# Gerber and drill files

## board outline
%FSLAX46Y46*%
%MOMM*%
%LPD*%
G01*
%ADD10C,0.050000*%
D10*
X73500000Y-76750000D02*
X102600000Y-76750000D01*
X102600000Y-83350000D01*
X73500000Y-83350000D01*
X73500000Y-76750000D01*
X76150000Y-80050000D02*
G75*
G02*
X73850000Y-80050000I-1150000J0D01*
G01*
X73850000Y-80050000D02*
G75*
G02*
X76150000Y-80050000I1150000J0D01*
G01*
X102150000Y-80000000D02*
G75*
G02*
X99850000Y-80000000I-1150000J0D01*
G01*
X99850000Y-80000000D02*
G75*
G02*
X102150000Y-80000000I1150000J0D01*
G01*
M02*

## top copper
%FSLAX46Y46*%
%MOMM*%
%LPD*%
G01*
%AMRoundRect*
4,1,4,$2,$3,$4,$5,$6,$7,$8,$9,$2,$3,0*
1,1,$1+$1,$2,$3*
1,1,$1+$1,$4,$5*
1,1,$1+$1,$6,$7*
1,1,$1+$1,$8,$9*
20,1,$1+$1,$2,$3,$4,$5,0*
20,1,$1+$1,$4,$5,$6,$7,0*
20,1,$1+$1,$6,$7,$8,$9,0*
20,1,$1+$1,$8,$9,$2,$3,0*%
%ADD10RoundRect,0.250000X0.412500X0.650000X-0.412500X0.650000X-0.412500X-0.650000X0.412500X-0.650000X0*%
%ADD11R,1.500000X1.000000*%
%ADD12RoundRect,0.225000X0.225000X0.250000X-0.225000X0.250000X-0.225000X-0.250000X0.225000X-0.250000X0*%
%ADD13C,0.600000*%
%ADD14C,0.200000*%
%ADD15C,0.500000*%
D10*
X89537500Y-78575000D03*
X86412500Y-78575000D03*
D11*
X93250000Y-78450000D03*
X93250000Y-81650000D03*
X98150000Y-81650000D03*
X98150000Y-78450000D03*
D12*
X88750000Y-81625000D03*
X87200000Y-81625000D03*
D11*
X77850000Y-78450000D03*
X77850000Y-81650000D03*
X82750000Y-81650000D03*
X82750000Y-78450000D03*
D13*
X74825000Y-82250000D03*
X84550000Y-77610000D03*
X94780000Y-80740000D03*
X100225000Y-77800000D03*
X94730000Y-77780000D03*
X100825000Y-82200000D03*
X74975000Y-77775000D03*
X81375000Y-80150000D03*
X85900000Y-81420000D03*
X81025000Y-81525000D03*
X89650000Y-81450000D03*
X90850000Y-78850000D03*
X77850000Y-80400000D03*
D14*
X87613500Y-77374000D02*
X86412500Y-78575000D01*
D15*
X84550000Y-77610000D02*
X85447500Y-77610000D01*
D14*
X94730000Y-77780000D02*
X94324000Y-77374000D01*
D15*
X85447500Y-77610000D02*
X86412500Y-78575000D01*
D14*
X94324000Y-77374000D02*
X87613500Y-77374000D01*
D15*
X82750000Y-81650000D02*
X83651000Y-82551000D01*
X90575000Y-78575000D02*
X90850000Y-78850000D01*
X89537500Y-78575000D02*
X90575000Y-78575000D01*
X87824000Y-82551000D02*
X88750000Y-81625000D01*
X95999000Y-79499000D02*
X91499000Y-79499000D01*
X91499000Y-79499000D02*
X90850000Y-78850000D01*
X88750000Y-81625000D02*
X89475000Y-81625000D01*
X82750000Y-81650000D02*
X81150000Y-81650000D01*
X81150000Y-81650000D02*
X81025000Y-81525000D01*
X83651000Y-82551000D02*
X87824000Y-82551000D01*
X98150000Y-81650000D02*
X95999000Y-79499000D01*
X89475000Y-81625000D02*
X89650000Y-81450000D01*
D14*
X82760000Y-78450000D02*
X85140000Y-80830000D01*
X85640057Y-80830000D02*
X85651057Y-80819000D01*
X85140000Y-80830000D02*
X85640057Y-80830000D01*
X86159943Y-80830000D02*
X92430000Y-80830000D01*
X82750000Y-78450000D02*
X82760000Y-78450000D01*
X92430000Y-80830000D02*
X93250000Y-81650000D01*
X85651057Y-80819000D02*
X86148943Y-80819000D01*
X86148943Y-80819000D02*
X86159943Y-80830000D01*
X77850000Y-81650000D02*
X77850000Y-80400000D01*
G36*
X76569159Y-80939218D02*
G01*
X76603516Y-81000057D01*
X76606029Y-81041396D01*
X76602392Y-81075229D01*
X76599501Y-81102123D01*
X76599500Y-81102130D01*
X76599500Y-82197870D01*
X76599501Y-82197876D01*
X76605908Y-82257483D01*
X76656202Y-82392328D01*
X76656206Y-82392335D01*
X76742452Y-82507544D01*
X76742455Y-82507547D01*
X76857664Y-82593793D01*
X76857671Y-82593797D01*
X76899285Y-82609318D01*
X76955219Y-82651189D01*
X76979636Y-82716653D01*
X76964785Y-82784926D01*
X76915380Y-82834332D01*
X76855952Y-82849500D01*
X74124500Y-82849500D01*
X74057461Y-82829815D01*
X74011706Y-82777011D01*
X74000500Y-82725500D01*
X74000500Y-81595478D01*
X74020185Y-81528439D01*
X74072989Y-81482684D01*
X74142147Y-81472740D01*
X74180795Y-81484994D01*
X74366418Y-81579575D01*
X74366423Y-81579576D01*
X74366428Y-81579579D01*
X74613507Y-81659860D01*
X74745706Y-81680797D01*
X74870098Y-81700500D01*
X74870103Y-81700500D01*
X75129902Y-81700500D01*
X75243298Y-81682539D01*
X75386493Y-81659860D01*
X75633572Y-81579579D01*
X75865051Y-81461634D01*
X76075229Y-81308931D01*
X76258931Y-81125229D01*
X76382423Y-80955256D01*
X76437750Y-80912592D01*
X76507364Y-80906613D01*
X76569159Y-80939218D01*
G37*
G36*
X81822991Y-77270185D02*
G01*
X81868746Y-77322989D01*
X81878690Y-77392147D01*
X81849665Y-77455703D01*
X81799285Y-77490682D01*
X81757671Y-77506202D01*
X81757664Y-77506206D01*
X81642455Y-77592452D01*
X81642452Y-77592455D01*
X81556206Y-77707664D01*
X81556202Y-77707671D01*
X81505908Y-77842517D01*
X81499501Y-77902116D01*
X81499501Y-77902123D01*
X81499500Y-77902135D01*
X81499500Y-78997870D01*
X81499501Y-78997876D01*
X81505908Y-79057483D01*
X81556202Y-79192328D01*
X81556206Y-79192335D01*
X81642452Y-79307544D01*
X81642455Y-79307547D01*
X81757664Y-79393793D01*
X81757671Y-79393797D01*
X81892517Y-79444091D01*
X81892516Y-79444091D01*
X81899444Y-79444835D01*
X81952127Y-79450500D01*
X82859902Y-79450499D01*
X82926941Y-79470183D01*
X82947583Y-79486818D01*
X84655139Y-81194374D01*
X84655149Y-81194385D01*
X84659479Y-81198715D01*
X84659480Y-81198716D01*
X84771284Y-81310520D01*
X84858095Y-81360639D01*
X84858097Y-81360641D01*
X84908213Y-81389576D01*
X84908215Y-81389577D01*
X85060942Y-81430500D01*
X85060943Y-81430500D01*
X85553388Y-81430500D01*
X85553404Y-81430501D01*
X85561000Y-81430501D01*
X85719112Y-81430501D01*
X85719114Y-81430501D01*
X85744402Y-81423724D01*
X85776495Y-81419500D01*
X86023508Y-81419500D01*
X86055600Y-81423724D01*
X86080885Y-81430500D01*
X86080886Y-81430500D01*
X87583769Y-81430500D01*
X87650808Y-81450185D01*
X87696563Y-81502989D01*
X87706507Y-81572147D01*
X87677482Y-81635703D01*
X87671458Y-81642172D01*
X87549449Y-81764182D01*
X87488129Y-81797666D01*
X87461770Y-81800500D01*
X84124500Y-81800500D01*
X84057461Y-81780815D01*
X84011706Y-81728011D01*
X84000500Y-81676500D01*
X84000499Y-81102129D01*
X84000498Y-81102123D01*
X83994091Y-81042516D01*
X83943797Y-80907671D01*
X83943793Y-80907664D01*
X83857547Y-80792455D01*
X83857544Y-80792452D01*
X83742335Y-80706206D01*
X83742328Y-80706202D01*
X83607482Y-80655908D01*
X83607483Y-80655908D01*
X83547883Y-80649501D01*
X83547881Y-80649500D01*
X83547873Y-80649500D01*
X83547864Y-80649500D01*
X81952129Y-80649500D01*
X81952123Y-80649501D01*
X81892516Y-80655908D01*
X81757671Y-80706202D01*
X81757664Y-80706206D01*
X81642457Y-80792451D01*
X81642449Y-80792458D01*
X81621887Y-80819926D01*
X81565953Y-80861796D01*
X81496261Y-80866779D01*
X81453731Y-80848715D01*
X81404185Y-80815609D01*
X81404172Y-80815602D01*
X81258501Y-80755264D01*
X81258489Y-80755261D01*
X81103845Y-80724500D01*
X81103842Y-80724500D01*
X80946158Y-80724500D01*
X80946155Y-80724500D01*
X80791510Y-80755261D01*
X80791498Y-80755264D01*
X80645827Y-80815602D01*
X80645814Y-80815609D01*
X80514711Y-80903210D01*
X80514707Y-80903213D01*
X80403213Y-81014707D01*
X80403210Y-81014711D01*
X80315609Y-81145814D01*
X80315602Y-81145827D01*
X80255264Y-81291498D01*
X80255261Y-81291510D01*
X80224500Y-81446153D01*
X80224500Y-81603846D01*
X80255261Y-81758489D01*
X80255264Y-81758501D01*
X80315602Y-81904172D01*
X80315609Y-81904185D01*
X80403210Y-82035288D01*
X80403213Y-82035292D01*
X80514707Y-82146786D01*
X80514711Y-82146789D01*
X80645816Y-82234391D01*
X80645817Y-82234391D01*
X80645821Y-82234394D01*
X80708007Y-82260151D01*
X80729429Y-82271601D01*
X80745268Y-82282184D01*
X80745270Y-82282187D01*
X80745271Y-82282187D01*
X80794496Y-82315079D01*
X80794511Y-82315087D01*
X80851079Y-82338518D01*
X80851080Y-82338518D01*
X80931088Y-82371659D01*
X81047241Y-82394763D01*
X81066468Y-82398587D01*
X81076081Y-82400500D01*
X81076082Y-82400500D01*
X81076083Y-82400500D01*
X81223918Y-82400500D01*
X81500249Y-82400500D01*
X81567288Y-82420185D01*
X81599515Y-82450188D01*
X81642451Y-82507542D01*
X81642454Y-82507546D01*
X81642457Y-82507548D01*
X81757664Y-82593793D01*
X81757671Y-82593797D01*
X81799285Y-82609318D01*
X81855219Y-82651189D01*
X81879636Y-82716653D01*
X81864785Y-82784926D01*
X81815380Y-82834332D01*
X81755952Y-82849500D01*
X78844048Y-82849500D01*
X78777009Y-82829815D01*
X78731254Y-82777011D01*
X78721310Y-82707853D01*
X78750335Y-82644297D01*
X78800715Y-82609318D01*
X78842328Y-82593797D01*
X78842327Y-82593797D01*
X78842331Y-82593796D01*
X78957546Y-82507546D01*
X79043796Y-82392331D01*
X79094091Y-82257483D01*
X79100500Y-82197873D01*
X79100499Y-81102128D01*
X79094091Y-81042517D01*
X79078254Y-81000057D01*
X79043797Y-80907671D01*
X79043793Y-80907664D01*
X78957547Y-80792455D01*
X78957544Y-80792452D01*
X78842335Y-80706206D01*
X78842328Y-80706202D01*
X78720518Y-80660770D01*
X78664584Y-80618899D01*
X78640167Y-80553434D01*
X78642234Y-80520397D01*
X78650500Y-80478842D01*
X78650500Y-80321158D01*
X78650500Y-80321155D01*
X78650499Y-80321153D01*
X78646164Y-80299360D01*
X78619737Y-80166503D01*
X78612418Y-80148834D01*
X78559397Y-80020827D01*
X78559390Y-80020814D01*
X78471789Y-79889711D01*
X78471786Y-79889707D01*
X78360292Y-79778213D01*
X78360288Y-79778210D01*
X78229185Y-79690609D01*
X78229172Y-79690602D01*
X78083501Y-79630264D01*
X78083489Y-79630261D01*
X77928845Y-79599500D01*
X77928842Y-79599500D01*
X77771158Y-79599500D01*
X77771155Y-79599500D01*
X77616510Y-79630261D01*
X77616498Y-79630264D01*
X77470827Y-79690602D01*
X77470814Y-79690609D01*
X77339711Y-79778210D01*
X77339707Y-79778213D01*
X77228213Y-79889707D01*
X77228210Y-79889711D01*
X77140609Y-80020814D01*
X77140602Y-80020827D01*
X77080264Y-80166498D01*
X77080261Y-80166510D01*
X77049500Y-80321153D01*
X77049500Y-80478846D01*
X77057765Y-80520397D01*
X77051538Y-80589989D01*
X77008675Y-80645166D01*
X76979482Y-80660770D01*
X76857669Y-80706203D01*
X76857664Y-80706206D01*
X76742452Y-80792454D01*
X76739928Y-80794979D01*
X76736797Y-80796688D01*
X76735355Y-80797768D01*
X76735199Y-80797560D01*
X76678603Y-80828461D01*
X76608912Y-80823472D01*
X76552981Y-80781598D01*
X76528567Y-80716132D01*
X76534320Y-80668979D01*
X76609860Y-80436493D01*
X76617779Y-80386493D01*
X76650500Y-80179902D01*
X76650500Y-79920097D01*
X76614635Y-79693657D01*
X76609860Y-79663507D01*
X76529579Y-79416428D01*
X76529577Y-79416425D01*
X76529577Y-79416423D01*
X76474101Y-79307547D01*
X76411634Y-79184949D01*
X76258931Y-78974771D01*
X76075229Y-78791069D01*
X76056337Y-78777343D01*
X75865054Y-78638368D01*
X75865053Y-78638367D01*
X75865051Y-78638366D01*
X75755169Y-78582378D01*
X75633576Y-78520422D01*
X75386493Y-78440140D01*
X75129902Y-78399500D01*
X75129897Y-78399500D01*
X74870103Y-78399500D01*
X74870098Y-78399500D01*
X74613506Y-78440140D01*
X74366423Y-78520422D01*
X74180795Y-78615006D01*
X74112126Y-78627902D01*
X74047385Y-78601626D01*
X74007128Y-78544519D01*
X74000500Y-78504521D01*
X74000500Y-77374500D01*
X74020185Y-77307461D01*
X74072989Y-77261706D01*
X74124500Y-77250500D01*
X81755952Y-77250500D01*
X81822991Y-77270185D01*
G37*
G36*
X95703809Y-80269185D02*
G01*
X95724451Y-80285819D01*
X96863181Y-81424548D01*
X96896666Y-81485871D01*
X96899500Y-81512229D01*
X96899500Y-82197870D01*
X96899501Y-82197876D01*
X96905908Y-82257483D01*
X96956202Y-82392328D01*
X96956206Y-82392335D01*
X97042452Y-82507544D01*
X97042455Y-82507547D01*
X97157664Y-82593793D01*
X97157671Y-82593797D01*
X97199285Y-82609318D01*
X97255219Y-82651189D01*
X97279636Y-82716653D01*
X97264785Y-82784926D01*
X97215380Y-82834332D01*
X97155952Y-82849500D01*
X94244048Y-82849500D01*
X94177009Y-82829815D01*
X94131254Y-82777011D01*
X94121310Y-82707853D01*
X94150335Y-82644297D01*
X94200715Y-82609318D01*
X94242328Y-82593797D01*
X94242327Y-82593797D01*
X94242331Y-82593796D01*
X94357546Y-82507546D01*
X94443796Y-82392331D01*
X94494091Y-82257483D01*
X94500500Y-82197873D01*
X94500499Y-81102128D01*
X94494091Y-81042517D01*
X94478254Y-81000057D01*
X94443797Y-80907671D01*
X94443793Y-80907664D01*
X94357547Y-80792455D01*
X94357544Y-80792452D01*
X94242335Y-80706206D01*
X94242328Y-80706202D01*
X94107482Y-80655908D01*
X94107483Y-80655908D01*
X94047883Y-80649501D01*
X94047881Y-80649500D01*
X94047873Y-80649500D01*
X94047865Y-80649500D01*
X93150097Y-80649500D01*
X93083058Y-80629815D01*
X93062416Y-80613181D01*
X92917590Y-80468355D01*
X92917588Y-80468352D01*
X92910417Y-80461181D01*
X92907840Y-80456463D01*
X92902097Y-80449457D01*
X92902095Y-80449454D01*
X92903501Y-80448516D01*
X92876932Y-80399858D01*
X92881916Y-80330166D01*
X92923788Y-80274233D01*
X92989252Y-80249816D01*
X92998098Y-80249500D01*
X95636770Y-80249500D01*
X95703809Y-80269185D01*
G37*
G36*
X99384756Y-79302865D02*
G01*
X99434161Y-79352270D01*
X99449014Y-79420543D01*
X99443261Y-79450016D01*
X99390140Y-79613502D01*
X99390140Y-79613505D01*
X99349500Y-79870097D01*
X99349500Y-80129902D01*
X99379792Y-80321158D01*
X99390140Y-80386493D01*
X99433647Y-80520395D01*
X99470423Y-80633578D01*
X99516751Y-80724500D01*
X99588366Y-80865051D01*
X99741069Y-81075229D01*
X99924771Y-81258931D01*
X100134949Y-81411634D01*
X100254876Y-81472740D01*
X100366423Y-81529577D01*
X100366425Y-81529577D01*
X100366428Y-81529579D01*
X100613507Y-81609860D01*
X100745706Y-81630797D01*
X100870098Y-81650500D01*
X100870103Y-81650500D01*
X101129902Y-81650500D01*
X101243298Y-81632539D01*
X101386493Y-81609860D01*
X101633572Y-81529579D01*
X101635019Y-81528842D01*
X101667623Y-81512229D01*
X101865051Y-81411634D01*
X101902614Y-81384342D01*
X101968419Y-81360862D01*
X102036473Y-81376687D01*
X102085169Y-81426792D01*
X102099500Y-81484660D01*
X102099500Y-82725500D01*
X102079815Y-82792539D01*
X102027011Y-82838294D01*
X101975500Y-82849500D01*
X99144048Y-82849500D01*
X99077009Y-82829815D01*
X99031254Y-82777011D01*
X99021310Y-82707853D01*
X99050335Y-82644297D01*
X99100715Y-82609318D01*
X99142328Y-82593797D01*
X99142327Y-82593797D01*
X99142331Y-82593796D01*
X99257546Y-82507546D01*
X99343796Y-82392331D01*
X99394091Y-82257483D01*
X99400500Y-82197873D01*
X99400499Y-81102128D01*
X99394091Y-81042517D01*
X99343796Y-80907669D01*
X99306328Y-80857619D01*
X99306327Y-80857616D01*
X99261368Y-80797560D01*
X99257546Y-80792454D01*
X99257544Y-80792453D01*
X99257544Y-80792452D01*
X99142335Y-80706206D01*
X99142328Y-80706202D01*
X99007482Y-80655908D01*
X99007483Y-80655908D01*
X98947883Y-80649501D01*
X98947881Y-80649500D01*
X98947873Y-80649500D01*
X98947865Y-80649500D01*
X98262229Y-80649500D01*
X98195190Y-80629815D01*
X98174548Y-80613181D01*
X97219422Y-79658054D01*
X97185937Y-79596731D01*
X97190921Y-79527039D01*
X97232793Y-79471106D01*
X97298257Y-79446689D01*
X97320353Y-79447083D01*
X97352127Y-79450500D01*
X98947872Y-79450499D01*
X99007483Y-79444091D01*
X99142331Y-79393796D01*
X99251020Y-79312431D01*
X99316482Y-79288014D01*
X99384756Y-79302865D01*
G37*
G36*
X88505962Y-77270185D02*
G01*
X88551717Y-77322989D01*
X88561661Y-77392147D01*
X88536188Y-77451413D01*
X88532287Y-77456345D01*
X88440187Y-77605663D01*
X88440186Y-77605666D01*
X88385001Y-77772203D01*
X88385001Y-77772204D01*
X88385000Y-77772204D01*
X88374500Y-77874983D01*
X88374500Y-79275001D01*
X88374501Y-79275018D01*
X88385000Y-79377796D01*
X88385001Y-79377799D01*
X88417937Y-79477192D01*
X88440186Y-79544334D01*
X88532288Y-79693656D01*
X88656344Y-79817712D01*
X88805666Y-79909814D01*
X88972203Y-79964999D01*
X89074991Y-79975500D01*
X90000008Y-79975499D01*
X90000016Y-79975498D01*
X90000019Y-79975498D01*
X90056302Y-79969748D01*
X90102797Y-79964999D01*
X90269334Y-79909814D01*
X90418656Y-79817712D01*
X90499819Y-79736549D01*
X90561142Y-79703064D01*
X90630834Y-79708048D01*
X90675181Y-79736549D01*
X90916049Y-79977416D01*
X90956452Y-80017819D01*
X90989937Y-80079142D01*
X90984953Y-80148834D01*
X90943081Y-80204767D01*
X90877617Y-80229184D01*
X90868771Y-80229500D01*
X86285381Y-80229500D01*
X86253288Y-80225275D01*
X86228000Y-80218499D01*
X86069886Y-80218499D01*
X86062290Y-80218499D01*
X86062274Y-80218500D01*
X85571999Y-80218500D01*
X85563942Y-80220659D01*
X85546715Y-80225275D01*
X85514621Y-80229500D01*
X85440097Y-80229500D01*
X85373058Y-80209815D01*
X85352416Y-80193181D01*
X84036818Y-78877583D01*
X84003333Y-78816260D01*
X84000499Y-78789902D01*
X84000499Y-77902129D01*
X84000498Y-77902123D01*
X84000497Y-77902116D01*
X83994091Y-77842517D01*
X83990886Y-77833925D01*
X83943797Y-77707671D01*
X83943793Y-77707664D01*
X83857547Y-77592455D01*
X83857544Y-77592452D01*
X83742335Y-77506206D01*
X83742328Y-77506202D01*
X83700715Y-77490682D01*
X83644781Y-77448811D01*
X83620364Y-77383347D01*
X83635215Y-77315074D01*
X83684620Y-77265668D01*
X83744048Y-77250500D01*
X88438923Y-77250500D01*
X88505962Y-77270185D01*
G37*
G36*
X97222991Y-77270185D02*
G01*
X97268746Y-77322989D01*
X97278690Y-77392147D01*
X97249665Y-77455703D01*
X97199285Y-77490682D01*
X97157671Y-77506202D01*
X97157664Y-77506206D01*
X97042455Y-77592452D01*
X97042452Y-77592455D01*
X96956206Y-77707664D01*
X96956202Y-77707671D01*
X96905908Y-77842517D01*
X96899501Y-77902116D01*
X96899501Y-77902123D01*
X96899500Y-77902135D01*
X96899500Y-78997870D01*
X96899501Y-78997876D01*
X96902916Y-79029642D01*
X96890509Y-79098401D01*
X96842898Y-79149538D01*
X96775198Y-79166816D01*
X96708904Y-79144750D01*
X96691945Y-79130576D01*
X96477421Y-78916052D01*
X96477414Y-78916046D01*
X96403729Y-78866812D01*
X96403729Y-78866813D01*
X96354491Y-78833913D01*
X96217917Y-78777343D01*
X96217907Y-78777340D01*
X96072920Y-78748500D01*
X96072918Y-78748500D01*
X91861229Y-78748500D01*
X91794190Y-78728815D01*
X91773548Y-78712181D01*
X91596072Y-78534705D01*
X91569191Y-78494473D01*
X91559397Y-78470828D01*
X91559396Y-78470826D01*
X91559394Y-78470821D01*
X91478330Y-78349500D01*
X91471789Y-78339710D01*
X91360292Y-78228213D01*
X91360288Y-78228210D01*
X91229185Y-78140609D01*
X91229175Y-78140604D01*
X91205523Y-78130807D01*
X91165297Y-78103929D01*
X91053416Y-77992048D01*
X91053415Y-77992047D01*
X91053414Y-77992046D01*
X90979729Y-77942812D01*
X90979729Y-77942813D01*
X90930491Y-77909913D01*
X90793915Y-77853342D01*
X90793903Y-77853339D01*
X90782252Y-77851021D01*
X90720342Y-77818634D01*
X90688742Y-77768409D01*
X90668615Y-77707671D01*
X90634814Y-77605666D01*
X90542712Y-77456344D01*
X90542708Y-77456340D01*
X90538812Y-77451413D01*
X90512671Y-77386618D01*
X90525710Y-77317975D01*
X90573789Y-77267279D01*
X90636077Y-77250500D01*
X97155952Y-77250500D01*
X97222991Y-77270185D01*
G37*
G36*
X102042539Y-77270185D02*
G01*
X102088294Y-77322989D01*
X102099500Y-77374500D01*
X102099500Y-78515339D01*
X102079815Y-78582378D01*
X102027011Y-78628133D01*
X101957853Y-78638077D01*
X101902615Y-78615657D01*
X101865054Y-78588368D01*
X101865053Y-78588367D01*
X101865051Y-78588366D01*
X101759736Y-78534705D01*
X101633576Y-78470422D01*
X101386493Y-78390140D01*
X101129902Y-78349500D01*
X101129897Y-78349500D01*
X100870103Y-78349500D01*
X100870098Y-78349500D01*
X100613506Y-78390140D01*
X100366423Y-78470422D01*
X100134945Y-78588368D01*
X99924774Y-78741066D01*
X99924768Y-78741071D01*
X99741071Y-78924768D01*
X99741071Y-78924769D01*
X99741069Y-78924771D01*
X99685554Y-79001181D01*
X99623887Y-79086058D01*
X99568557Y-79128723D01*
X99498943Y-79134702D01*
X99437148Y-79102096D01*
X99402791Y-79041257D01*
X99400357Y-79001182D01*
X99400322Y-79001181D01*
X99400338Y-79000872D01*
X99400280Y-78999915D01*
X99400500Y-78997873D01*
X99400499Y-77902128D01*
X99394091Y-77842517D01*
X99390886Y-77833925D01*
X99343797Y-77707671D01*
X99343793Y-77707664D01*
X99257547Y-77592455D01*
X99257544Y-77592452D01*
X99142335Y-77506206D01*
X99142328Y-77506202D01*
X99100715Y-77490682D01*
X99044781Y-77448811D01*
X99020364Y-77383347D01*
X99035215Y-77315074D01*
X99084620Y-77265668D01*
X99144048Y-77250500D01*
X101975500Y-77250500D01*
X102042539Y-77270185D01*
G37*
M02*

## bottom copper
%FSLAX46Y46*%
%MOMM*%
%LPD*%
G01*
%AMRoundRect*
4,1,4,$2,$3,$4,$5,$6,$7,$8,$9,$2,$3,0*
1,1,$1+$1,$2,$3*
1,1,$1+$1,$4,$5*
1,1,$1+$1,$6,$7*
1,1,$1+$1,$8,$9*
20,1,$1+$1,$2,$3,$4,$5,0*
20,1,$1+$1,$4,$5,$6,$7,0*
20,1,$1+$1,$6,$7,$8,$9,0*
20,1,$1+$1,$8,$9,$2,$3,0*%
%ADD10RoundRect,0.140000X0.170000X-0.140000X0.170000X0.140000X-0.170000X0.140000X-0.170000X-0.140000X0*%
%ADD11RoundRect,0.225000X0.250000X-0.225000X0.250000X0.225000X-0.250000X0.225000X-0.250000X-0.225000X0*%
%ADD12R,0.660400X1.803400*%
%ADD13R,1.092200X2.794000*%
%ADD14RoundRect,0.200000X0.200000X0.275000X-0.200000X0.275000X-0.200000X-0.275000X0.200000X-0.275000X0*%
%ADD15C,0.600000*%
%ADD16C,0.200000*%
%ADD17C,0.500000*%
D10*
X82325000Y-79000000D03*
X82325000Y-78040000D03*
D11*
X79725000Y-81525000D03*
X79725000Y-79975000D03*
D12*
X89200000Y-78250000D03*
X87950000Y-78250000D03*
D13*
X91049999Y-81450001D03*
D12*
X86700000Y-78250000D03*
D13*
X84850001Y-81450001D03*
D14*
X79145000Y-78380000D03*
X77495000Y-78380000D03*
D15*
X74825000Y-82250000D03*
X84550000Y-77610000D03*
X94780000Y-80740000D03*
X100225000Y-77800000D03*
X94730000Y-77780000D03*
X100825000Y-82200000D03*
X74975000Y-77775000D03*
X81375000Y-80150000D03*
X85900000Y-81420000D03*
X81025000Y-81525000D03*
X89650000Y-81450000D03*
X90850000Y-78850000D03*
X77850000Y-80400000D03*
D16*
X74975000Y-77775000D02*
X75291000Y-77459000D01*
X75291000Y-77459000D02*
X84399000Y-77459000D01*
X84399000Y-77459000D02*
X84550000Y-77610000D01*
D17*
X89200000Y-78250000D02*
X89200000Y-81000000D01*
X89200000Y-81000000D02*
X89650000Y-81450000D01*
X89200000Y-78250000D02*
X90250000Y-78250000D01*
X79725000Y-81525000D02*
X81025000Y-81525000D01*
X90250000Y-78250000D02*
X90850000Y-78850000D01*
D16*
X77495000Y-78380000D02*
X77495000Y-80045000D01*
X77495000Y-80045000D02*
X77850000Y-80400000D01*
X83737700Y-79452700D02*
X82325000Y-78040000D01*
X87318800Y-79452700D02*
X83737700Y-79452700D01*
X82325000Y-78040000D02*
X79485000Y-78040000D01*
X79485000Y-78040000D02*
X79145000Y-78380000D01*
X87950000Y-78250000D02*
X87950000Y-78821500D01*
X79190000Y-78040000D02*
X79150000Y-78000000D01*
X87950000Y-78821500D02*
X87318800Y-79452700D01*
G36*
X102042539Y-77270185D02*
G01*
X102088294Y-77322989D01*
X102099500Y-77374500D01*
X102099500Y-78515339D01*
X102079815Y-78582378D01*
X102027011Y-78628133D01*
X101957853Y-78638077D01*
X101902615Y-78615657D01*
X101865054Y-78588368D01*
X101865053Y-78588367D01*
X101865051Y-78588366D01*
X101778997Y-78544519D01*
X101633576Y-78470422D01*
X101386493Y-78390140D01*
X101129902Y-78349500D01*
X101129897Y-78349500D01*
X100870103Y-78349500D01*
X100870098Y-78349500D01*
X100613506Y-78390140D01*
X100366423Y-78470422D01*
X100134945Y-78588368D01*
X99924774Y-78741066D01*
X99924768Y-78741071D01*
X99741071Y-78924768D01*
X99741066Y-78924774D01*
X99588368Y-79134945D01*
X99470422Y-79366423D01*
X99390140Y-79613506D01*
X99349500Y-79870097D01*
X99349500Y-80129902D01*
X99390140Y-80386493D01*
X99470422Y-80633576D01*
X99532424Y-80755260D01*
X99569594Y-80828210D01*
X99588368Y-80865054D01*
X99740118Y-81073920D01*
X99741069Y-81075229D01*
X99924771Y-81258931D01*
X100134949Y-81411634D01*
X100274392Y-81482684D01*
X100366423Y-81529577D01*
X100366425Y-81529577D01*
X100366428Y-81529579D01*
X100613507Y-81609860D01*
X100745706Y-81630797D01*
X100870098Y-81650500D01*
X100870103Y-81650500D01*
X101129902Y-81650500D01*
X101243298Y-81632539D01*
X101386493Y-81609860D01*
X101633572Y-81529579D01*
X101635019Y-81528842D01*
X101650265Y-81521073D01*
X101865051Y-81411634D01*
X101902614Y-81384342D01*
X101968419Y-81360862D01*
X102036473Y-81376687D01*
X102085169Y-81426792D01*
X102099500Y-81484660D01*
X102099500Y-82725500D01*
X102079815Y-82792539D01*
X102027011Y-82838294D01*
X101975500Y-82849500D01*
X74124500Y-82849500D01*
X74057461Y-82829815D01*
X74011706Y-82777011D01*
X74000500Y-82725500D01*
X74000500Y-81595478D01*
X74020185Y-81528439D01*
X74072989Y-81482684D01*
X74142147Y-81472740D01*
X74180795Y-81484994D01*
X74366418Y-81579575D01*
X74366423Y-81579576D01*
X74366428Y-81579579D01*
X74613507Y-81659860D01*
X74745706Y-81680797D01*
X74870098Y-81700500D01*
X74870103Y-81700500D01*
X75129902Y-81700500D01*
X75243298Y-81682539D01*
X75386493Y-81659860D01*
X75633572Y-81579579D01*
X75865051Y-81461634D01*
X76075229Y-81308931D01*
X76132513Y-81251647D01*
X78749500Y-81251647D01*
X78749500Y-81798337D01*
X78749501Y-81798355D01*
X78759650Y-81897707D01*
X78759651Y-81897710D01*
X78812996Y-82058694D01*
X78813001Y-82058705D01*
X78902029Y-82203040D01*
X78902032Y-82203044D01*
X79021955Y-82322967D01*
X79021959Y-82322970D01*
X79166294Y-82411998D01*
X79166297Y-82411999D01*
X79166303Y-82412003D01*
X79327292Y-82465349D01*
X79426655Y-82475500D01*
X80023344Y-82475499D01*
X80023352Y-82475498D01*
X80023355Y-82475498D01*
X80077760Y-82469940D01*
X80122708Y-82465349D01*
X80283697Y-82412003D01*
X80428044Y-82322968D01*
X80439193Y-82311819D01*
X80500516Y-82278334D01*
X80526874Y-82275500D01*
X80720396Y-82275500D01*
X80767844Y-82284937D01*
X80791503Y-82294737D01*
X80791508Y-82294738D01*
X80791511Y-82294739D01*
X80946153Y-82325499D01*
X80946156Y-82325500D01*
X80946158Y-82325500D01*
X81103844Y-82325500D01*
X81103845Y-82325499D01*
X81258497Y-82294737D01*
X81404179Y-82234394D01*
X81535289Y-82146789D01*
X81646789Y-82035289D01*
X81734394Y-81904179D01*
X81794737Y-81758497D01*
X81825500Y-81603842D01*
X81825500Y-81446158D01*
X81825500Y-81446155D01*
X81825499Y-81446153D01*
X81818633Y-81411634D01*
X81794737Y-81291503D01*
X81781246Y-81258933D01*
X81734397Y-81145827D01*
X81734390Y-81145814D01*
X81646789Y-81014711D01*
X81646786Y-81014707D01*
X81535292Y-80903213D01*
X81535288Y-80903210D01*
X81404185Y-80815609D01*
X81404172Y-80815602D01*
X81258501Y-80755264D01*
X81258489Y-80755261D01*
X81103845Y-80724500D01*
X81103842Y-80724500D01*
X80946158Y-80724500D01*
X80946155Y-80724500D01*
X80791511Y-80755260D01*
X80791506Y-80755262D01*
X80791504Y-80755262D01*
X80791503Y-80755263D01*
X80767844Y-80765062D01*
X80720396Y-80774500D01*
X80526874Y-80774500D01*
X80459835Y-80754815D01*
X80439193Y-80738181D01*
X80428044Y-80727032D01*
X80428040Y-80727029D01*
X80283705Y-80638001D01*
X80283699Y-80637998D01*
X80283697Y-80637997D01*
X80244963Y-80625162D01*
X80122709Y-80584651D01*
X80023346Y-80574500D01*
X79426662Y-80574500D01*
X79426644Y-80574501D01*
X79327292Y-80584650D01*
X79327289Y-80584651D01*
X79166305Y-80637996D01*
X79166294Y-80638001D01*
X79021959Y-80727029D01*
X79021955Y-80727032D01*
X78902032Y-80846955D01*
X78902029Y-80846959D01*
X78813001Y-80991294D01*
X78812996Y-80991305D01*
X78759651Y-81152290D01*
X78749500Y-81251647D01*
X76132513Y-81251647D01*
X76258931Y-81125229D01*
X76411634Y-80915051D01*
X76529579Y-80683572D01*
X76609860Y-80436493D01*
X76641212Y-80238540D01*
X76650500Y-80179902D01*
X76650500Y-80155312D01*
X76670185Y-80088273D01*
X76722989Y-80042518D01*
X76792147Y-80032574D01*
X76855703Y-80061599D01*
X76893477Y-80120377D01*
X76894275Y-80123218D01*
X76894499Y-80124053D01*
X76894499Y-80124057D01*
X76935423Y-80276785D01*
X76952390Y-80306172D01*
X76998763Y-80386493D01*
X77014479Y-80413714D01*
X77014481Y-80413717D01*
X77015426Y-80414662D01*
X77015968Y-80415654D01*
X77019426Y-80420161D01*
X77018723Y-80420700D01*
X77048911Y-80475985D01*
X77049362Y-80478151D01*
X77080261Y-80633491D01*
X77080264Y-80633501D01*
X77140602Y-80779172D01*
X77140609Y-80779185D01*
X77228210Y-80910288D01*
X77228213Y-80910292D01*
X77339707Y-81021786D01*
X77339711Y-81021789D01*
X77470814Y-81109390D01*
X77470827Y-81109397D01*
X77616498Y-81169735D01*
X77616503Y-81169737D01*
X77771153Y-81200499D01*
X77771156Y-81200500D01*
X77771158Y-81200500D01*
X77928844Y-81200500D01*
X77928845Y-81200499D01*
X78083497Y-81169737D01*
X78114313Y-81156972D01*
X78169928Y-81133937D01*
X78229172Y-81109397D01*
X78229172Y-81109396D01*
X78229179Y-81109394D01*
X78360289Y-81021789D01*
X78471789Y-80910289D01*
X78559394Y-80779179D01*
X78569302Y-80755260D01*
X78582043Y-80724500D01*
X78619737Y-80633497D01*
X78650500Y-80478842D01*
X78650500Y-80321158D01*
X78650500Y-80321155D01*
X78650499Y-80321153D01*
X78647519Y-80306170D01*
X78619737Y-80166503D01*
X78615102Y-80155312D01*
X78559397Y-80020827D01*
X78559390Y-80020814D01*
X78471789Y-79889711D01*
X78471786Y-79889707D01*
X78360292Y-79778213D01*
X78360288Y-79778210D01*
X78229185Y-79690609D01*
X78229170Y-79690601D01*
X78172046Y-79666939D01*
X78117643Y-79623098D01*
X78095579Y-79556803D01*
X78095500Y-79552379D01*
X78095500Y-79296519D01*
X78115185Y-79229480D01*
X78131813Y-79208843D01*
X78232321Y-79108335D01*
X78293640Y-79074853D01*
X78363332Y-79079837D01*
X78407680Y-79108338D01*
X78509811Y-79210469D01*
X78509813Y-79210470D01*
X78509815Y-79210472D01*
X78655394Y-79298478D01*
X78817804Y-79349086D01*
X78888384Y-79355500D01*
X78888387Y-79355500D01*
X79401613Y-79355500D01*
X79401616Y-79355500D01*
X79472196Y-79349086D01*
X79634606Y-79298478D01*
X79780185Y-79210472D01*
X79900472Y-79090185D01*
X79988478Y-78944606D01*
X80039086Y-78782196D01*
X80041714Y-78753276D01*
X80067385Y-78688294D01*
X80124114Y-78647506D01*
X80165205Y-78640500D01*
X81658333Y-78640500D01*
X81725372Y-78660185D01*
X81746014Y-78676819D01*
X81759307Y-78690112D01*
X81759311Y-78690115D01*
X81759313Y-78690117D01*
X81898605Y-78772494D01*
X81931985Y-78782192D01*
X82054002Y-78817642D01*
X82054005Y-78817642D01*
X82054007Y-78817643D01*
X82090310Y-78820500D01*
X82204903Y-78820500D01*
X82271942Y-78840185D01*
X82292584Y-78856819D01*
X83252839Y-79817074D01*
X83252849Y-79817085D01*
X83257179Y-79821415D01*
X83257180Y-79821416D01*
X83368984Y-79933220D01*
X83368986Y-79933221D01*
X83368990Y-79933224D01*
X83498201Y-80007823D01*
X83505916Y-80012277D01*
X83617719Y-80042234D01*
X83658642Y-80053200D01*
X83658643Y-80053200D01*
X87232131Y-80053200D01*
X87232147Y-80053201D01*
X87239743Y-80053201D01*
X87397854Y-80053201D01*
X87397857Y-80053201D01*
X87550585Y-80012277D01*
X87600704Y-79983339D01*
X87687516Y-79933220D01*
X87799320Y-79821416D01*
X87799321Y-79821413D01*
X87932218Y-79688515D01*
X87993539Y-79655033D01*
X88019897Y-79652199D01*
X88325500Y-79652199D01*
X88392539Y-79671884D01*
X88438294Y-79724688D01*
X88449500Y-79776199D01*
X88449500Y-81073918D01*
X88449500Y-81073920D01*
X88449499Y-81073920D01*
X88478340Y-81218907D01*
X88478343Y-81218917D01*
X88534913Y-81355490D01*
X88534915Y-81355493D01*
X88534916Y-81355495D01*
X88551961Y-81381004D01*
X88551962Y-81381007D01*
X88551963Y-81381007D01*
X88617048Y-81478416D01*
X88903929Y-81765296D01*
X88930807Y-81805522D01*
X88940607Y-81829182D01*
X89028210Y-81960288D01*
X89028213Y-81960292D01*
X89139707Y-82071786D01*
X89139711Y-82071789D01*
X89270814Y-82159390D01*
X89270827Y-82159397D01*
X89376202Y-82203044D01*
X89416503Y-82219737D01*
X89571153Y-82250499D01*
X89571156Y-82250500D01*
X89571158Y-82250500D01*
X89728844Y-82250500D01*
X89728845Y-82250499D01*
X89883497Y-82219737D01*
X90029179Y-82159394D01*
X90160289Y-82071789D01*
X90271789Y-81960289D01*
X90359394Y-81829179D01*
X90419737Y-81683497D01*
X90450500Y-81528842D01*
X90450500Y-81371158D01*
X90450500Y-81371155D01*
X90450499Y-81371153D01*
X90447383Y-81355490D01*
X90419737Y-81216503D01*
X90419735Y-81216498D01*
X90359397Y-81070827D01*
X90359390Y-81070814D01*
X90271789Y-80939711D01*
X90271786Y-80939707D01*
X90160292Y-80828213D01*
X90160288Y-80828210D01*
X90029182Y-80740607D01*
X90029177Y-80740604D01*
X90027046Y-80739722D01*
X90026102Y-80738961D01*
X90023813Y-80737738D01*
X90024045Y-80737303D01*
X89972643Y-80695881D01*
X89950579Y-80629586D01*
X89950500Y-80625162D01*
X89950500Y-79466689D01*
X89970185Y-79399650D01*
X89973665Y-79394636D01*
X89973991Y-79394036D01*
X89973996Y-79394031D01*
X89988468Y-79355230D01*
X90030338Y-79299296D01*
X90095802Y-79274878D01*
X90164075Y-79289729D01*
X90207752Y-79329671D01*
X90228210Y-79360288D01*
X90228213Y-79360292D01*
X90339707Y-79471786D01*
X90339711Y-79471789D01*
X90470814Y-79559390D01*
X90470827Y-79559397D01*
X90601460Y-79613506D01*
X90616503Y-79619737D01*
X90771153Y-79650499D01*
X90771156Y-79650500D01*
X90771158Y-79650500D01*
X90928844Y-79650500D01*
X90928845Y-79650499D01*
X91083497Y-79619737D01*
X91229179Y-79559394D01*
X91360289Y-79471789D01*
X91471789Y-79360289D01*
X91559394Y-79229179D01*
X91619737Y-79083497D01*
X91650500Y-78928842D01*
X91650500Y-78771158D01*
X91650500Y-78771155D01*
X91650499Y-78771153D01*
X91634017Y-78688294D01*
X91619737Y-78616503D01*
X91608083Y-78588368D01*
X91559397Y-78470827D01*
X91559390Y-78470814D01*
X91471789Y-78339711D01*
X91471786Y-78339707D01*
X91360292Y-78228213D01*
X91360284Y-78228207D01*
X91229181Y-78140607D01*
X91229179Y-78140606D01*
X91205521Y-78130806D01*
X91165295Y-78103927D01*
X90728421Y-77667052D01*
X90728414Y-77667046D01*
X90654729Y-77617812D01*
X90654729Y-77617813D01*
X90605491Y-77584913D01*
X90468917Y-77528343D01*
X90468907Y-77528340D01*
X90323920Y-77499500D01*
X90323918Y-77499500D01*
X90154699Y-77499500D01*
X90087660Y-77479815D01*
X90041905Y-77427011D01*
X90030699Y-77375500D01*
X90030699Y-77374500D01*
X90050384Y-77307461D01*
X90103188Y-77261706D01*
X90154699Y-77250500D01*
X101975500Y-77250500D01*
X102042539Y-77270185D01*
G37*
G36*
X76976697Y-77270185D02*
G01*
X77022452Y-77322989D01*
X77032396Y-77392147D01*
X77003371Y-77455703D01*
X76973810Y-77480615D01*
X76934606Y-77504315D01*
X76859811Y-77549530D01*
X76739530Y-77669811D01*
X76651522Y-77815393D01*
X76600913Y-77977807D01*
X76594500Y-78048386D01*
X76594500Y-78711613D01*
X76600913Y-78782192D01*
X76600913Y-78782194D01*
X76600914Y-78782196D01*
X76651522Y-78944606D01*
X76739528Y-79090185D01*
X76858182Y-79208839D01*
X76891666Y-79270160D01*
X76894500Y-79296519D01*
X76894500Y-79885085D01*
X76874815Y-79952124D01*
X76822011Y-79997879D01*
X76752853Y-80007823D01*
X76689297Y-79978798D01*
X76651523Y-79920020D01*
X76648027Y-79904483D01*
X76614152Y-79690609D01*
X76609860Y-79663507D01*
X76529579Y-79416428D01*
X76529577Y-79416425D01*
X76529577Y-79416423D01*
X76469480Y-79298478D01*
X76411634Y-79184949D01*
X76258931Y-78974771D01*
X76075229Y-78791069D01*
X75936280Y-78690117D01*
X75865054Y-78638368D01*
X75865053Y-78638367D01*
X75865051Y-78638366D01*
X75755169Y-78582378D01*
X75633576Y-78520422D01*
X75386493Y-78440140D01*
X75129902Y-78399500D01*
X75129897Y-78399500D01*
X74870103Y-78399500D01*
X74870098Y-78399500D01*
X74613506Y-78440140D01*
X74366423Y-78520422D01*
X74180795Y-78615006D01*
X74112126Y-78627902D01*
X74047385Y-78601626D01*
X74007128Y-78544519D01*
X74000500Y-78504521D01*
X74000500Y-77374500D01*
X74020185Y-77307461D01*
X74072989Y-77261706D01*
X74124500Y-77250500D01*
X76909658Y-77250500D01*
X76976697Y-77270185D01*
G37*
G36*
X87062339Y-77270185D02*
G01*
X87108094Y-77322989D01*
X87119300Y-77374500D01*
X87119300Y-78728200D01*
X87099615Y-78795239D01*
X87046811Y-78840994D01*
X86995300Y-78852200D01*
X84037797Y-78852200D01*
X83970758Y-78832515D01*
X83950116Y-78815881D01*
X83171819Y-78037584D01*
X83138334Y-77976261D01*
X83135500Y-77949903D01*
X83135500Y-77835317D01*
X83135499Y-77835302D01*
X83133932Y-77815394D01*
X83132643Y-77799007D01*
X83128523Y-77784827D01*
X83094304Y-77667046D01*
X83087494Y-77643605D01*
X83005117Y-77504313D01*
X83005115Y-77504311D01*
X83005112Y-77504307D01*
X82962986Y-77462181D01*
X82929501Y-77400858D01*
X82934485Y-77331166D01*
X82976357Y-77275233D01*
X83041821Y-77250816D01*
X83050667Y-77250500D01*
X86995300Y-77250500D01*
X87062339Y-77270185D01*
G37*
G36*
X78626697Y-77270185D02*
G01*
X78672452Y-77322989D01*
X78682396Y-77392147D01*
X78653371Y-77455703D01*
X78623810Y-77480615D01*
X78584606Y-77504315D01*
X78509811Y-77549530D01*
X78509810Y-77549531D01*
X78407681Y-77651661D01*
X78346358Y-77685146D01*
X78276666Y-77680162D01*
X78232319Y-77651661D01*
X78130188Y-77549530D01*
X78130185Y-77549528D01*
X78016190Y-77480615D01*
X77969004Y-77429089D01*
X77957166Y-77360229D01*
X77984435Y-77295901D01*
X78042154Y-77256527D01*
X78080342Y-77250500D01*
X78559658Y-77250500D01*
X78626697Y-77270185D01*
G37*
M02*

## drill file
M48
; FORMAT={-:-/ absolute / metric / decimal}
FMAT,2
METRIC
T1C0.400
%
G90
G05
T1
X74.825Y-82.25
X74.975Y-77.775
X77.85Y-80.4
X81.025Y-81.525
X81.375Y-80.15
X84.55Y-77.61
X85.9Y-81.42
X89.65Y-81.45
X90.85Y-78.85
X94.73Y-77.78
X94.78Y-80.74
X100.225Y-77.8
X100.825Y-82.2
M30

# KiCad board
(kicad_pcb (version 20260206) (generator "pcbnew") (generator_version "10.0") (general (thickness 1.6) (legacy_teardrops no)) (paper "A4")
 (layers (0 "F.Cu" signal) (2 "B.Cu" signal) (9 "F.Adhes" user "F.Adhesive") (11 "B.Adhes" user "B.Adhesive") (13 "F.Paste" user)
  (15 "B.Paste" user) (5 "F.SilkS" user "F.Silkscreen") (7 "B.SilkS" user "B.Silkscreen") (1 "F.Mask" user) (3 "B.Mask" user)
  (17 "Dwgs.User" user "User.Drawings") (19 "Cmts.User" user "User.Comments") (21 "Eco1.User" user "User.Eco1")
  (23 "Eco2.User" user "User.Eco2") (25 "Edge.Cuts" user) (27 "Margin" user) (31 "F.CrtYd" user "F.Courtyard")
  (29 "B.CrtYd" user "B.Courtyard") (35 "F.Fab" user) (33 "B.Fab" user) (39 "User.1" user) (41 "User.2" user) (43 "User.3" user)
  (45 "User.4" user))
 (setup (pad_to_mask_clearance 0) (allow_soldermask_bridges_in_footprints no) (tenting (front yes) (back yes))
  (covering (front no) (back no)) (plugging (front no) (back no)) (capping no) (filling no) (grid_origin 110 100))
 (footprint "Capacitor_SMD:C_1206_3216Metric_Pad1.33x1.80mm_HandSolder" (layer "F.Cu") (at 87.975 78.575 180)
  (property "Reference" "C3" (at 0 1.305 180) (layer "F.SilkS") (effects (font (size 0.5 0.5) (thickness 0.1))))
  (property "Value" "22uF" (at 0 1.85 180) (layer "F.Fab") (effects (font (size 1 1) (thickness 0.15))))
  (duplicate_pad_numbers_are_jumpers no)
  (pad "1" smd roundrect (at -1.5625 0 180) (size 1.325 1.8) (layers "F.Cu" "F.Mask" "F.Paste") (roundrect_rratio 0.188679) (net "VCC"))
  (pad "2" smd roundrect (at 1.5625 0 180) (size 1.325 1.8) (layers "F.Cu" "F.Mask" "F.Paste") (roundrect_rratio 0.188679) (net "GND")))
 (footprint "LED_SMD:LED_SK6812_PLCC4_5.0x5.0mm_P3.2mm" (layer "F.Cu") (at 95.7 80.05)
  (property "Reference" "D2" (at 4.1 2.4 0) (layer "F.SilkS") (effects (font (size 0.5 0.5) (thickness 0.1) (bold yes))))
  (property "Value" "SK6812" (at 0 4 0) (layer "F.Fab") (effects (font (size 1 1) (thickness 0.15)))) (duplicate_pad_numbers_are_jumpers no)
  (pad "1" smd rect (at -2.45 -1.6 180) (size 1.5 1) (layers "F.Cu" "F.Mask" "F.Paste") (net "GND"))
  (pad "2" smd rect (at -2.45 1.6 180) (size 1.5 1) (layers "F.Cu" "F.Mask" "F.Paste") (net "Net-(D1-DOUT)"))
  (pad "3" smd rect (at 2.45 1.6 180) (size 1.5 1) (layers "F.Cu" "F.Mask" "F.Paste") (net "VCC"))
  (pad "4" smd rect (at 2.45 -1.6 180) (size 1.5 1) (layers "F.Cu" "F.Mask" "F.Paste") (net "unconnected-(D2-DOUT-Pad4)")))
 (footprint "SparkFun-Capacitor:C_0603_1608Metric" (layer "F.Cu") (at 87.975 81.625 180)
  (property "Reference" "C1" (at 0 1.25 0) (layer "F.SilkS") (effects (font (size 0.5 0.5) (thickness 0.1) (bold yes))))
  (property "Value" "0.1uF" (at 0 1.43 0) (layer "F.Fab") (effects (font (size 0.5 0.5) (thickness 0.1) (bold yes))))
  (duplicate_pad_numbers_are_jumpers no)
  (pad "1" smd roundrect (at -0.775 0 180) (size 0.9 0.95) (layers "F.Cu" "F.Mask" "F.Paste") (roundrect_rratio 0.25) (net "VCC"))
  (pad "2" smd roundrect (at 0.775 0 180) (size 0.9 0.95) (layers "F.Cu" "F.Mask" "F.Paste") (roundrect_rratio 0.25) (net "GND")))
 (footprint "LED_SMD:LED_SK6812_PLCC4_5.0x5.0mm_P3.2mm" (layer "F.Cu") (at 80.3 80.05)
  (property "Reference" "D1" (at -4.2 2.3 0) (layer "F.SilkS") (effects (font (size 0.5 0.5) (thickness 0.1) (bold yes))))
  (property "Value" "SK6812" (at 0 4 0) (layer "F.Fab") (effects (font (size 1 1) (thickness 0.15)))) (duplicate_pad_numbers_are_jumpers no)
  (pad "1" smd rect (at -2.45 -1.6 180) (size 1.5 1) (layers "F.Cu" "F.Mask" "F.Paste") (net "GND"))
  (pad "2" smd rect (at -2.45 1.6 180) (size 1.5 1) (layers "F.Cu" "F.Mask" "F.Paste") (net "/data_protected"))
  (pad "3" smd rect (at 2.45 1.6 180) (size 1.5 1) (layers "F.Cu" "F.Mask" "F.Paste") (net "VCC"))
  (pad "4" smd rect (at 2.45 -1.6 180) (size 1.5 1) (layers "F.Cu" "F.Mask" "F.Paste") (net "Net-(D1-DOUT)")))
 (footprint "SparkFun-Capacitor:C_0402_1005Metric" (layer "B.Cu") (at 82.325 78.52 90)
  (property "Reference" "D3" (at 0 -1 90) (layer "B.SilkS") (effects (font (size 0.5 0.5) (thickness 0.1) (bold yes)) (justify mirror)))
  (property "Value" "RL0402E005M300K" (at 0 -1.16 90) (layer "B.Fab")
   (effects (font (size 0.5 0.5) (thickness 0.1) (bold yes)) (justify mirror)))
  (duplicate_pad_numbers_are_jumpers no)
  (pad "1" smd roundrect (at -0.48 0 90) (size 0.56 0.62) (layers "B.Cu" "B.Mask" "B.Paste") (roundrect_rratio 0.25) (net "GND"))
  (pad "2" smd roundrect (at 0.48 0 90) (size 0.56 0.62) (layers "B.Cu" "B.Mask" "B.Paste") (roundrect_rratio 0.25) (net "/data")))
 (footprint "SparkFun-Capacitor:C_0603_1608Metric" (layer "B.Cu") (at 79.725 80.75 90)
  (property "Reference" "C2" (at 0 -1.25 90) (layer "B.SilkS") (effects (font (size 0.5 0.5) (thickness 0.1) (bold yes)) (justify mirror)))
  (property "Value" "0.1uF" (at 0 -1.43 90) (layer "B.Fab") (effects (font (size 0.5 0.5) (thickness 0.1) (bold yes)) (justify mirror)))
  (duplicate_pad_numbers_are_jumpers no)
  (pad "1" smd roundrect (at -0.775 0 90) (size 0.9 0.95) (layers "B.Cu" "B.Mask" "B.Paste") (roundrect_rratio 0.25) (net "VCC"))
  (pad "2" smd roundrect (at 0.775 0 90) (size 0.9 0.95) (layers "B.Cu" "B.Mask" "B.Paste") (roundrect_rratio 0.25) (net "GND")))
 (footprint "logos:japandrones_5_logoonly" (layer "B.Cu") (at 95.848759 79.08709 180)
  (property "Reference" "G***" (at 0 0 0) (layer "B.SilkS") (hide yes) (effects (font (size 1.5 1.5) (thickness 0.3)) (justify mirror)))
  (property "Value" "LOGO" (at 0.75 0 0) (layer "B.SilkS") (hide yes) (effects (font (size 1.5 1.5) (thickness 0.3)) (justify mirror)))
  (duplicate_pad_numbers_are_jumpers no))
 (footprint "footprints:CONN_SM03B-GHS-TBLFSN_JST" (layer "B.Cu") (at 87.95 80.453704 180)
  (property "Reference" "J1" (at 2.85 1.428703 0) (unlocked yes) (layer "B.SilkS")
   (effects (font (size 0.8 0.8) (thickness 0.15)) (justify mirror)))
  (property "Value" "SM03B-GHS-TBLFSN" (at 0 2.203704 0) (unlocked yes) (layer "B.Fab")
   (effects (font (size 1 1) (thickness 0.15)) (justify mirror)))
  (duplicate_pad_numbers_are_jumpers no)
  (pad "1" smd rect (at -1.25 2.203704 180) (size 0.6604 1.8034) (layers "B.Cu" "B.Mask" "B.Paste") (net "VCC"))
  (pad "2" smd rect (at 0 2.203704 180) (size 0.6604 1.8034) (layers "B.Cu" "B.Mask" "B.Paste") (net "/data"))
  (pad "3" smd rect (at -3.099999 -0.996297 180) (size 1.0922 2.794) (layers "B.Cu" "B.Mask" "B.Paste") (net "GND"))
  (pad "3" smd rect (at 1.25 2.203704 180) (size 0.6604 1.8034) (layers "B.Cu" "B.Mask" "B.Paste") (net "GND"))
  (pad "3" smd rect (at 3.099999 -0.996297 180) (size 1.0922 2.794) (layers "B.Cu" "B.Mask" "B.Paste") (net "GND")))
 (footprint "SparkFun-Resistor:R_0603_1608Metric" (layer "B.Cu") (at 78.32 78.38 180)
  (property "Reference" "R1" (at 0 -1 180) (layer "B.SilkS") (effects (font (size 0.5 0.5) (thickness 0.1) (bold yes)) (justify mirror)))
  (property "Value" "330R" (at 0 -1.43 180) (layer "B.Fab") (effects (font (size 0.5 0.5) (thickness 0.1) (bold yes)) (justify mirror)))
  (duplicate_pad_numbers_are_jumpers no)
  (pad "1" smd roundrect (at -0.825 0 180) (size 0.8 0.95) (layers "B.Cu" "B.Mask" "B.Paste") (roundrect_rratio 0.25) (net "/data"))
  (pad "2" smd roundrect (at 0.825 0 180) (size 0.8 0.95) (layers "B.Cu" "B.Mask" "B.Paste") (roundrect_rratio 0.25) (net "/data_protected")))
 (gr_rect (start 73.5 76.75) (end 102.6 83.35) (stroke (width 0.05) (type solid)) (fill no) (layer "Edge.Cuts"))
 (gr_circle (center 75 80.05) (end 76.15 80.05) (stroke (width 0.05) (type solid)) (fill no) (layer "Edge.Cuts"))
 (gr_circle (center 101 80) (end 102.15 80) (stroke (width 0.05) (type solid)) (fill no) (layer "Edge.Cuts"))
 (segment (start 87.6135 77.374) (end 86.4125 78.575) (width 0.2) (layer "F.Cu") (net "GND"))
 (segment (start 84.55 77.61) (end 85.4475 77.61) (width 0.5) (layer "F.Cu") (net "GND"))
 (segment (start 94.73 77.78) (end 94.324 77.374) (width 0.2) (layer "F.Cu") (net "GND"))
 (segment (start 85.4475 77.61) (end 86.4125 78.575) (width 0.5) (layer "F.Cu") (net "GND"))
 (segment (start 94.324 77.374) (end 87.6135 77.374) (width 0.2) (layer "F.Cu") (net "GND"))
 (via (at 74.825 82.25) (size 0.6) (drill 0.4) (layers "F.Cu" "B.Cu") (free yes) (capping no) (covering (front no) (back no))
  (plugging (front no) (back no)) (filling no) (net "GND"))
 (via (at 84.55 77.61) (size 0.6) (drill 0.4) (layers "F.Cu" "B.Cu") (free yes) (capping no) (covering (front no) (back no))
  (plugging (front no) (back no)) (filling no) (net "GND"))
 (via (at 94.78 80.74) (size 0.6) (drill 0.4) (layers "F.Cu" "B.Cu") (free yes) (capping no) (covering (front no) (back no))
  (plugging (front no) (back no)) (filling no) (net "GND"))
 (via (at 100.225 77.8) (size 0.6) (drill 0.4) (layers "F.Cu" "B.Cu") (free yes) (capping no) (covering (front no) (back no))
  (plugging (front no) (back no)) (filling no) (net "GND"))
 (via (at 94.73 77.78) (size 0.6) (drill 0.4) (layers "F.Cu" "B.Cu") (free yes) (capping no) (covering (front no) (back no))
  (plugging (front no) (back no)) (filling no) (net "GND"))
 (via (at 100.825 82.2) (size 0.6) (drill 0.4) (layers "F.Cu" "B.Cu") (free yes) (capping no) (covering (front no) (back no))
  (plugging (front no) (back no)) (filling no) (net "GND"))
 (via (at 74.975 77.775) (size 0.6) (drill 0.4) (layers "F.Cu" "B.Cu") (free yes) (capping no) (covering (front no) (back no))
  (plugging (front no) (back no)) (filling no) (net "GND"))
 (via (at 81.375 80.15) (size 0.6) (drill 0.4) (layers "F.Cu" "B.Cu") (free yes) (capping no) (covering (front no) (back no))
  (plugging (front no) (back no)) (filling no) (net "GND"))
 (via (at 85.9 81.42) (size 0.6) (drill 0.4) (layers "F.Cu" "B.Cu") (free yes) (capping no) (covering (front no) (back no))
  (plugging (front no) (back no)) (filling no) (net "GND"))
 (segment (start 74.975 77.775) (end 75.291 77.459) (width 0.2) (layer "B.Cu") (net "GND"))
 (segment (start 75.291 77.459) (end 84.399 77.459) (width 0.2) (layer "B.Cu") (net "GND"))
 (segment (start 84.399 77.459) (end 84.55 77.61) (width 0.2) (layer "B.Cu") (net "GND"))
 (segment (start 82.75 81.65) (end 83.651 82.551) (width 0.5) (layer "F.Cu") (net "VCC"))
 (segment (start 90.575 78.575) (end 90.85 78.85) (width 0.5) (layer "F.Cu") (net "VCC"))
 (segment (start 89.5375 78.575) (end 90.575 78.575) (width 0.5) (layer "F.Cu") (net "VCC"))
 (segment (start 87.824 82.551) (end 88.75 81.625) (width 0.5) (layer "F.Cu") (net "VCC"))
 (segment (start 95.999 79.499) (end 91.499 79.499) (width 0.5) (layer "F.Cu") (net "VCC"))
 (segment (start 91.499 79.499) (end 90.85 78.85) (width 0.5) (layer "F.Cu") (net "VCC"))
 (segment (start 88.75 81.625) (end 89.475 81.625) (width 0.5) (layer "F.Cu") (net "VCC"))
 (segment (start 82.75 81.65) (end 81.15 81.65) (width 0.5) (layer "F.Cu") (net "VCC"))
 (segment (start 81.15 81.65) (end 81.025 81.525) (width 0.5) (layer "F.Cu") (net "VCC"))
 (segment (start 83.651 82.551) (end 87.824 82.551) (width 0.5) (layer "F.Cu") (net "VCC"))
 (segment (start 98.15 81.65) (end 95.999 79.499) (width 0.5) (layer "F.Cu") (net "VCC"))
 (segment (start 89.475 81.625) (end 89.65 81.45) (width 0.5) (layer "F.Cu") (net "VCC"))
 (via (at 81.025 81.525) (size 0.6) (drill 0.4) (layers "F.Cu" "B.Cu") (capping no) (covering (front no) (back no))
  (plugging (front no) (back no)) (filling no) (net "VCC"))
 (via (at 89.65 81.45) (size 0.6) (drill 0.4) (layers "F.Cu" "B.Cu") (capping no) (covering (front no) (back no))
  (plugging (front no) (back no)) (filling no) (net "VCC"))
 (via (at 90.85 78.85) (size 0.6) (drill 0.4) (layers "F.Cu" "B.Cu") (capping no) (covering (front no) (back no))
  (plugging (front no) (back no)) (filling no) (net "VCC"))
 (segment (start 89.2 78.25) (end 89.2 81) (width 0.5) (layer "B.Cu") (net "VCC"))
 (segment (start 89.2 81) (end 89.65 81.45) (width 0.5) (layer "B.Cu") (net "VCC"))
 (segment (start 89.2 78.25) (end 90.25 78.25) (width 0.5) (layer "B.Cu") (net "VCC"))
 (segment (start 79.725 81.525) (end 81.025 81.525) (width 0.5) (layer "B.Cu") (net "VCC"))
 (segment (start 90.25 78.25) (end 90.85 78.85) (width 0.5) (layer "B.Cu") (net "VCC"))
 (segment (start 82.76 78.45) (end 85.14 80.83) (width 0.2) (layer "F.Cu") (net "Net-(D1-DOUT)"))
 (segment (start 85.640057 80.83) (end 85.651057 80.819) (width 0.2) (layer "F.Cu") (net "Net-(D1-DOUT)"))
 (segment (start 85.14 80.83) (end 85.640057 80.83) (width 0.2) (layer "F.Cu") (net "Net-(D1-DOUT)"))
 (segment (start 86.159943 80.83) (end 92.43 80.83) (width 0.2) (layer "F.Cu") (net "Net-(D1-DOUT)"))
 (segment (start 82.75 78.45) (end 82.76 78.45) (width 0.2) (layer "F.Cu") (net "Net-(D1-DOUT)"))
 (segment (start 92.43 80.83) (end 93.25 81.65) (width 0.2) (layer "F.Cu") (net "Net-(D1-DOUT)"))
 (segment (start 85.651057 80.819) (end 86.148943 80.819) (width 0.2) (layer "F.Cu") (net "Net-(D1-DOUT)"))
 (segment (start 86.148943 80.819) (end 86.159943 80.83) (width 0.2) (layer "F.Cu") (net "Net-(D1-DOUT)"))
 (segment (start 77.85 81.65) (end 77.85 80.4) (width 0.2) (layer "F.Cu") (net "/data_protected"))
 (via (at 77.85 80.4) (size 0.6) (drill 0.4) (layers "F.Cu" "B.Cu") (capping no) (covering (front no) (back no))
  (plugging (front no) (back no)) (filling no) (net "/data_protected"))
 (segment (start 77.495 78.38) (end 77.495 80.045) (width 0.2) (layer "B.Cu") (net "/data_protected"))
 (segment (start 77.495 80.045) (end 77.85 80.4) (width 0.2) (layer "B.Cu") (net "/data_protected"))
 (segment (start 83.7377 79.4527) (end 82.325 78.04) (width 0.2) (layer "B.Cu") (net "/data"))
 (segment (start 87.3188 79.4527) (end 83.7377 79.4527) (width 0.2) (layer "B.Cu") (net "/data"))
 (segment (start 82.325 78.04) (end 79.485 78.04) (width 0.2) (layer "B.Cu") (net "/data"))
 (segment (start 79.485 78.04) (end 79.145 78.38) (width 0.2) (layer "B.Cu") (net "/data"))
 (segment (start 87.95 78.25) (end 87.95 78.8215) (width 0.2) (layer "B.Cu") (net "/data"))
 (segment (start 79.19 78.04) (end 79.15 78) (width 0.2) (layer "B.Cu") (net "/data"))
 (segment (start 87.95 78.8215) (end 87.3188 79.4527) (width 0.2) (layer "B.Cu") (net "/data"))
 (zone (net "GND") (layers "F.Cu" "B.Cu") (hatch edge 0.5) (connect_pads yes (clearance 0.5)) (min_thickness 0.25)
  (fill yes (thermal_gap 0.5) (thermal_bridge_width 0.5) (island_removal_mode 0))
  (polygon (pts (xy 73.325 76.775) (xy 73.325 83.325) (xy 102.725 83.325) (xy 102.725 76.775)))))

